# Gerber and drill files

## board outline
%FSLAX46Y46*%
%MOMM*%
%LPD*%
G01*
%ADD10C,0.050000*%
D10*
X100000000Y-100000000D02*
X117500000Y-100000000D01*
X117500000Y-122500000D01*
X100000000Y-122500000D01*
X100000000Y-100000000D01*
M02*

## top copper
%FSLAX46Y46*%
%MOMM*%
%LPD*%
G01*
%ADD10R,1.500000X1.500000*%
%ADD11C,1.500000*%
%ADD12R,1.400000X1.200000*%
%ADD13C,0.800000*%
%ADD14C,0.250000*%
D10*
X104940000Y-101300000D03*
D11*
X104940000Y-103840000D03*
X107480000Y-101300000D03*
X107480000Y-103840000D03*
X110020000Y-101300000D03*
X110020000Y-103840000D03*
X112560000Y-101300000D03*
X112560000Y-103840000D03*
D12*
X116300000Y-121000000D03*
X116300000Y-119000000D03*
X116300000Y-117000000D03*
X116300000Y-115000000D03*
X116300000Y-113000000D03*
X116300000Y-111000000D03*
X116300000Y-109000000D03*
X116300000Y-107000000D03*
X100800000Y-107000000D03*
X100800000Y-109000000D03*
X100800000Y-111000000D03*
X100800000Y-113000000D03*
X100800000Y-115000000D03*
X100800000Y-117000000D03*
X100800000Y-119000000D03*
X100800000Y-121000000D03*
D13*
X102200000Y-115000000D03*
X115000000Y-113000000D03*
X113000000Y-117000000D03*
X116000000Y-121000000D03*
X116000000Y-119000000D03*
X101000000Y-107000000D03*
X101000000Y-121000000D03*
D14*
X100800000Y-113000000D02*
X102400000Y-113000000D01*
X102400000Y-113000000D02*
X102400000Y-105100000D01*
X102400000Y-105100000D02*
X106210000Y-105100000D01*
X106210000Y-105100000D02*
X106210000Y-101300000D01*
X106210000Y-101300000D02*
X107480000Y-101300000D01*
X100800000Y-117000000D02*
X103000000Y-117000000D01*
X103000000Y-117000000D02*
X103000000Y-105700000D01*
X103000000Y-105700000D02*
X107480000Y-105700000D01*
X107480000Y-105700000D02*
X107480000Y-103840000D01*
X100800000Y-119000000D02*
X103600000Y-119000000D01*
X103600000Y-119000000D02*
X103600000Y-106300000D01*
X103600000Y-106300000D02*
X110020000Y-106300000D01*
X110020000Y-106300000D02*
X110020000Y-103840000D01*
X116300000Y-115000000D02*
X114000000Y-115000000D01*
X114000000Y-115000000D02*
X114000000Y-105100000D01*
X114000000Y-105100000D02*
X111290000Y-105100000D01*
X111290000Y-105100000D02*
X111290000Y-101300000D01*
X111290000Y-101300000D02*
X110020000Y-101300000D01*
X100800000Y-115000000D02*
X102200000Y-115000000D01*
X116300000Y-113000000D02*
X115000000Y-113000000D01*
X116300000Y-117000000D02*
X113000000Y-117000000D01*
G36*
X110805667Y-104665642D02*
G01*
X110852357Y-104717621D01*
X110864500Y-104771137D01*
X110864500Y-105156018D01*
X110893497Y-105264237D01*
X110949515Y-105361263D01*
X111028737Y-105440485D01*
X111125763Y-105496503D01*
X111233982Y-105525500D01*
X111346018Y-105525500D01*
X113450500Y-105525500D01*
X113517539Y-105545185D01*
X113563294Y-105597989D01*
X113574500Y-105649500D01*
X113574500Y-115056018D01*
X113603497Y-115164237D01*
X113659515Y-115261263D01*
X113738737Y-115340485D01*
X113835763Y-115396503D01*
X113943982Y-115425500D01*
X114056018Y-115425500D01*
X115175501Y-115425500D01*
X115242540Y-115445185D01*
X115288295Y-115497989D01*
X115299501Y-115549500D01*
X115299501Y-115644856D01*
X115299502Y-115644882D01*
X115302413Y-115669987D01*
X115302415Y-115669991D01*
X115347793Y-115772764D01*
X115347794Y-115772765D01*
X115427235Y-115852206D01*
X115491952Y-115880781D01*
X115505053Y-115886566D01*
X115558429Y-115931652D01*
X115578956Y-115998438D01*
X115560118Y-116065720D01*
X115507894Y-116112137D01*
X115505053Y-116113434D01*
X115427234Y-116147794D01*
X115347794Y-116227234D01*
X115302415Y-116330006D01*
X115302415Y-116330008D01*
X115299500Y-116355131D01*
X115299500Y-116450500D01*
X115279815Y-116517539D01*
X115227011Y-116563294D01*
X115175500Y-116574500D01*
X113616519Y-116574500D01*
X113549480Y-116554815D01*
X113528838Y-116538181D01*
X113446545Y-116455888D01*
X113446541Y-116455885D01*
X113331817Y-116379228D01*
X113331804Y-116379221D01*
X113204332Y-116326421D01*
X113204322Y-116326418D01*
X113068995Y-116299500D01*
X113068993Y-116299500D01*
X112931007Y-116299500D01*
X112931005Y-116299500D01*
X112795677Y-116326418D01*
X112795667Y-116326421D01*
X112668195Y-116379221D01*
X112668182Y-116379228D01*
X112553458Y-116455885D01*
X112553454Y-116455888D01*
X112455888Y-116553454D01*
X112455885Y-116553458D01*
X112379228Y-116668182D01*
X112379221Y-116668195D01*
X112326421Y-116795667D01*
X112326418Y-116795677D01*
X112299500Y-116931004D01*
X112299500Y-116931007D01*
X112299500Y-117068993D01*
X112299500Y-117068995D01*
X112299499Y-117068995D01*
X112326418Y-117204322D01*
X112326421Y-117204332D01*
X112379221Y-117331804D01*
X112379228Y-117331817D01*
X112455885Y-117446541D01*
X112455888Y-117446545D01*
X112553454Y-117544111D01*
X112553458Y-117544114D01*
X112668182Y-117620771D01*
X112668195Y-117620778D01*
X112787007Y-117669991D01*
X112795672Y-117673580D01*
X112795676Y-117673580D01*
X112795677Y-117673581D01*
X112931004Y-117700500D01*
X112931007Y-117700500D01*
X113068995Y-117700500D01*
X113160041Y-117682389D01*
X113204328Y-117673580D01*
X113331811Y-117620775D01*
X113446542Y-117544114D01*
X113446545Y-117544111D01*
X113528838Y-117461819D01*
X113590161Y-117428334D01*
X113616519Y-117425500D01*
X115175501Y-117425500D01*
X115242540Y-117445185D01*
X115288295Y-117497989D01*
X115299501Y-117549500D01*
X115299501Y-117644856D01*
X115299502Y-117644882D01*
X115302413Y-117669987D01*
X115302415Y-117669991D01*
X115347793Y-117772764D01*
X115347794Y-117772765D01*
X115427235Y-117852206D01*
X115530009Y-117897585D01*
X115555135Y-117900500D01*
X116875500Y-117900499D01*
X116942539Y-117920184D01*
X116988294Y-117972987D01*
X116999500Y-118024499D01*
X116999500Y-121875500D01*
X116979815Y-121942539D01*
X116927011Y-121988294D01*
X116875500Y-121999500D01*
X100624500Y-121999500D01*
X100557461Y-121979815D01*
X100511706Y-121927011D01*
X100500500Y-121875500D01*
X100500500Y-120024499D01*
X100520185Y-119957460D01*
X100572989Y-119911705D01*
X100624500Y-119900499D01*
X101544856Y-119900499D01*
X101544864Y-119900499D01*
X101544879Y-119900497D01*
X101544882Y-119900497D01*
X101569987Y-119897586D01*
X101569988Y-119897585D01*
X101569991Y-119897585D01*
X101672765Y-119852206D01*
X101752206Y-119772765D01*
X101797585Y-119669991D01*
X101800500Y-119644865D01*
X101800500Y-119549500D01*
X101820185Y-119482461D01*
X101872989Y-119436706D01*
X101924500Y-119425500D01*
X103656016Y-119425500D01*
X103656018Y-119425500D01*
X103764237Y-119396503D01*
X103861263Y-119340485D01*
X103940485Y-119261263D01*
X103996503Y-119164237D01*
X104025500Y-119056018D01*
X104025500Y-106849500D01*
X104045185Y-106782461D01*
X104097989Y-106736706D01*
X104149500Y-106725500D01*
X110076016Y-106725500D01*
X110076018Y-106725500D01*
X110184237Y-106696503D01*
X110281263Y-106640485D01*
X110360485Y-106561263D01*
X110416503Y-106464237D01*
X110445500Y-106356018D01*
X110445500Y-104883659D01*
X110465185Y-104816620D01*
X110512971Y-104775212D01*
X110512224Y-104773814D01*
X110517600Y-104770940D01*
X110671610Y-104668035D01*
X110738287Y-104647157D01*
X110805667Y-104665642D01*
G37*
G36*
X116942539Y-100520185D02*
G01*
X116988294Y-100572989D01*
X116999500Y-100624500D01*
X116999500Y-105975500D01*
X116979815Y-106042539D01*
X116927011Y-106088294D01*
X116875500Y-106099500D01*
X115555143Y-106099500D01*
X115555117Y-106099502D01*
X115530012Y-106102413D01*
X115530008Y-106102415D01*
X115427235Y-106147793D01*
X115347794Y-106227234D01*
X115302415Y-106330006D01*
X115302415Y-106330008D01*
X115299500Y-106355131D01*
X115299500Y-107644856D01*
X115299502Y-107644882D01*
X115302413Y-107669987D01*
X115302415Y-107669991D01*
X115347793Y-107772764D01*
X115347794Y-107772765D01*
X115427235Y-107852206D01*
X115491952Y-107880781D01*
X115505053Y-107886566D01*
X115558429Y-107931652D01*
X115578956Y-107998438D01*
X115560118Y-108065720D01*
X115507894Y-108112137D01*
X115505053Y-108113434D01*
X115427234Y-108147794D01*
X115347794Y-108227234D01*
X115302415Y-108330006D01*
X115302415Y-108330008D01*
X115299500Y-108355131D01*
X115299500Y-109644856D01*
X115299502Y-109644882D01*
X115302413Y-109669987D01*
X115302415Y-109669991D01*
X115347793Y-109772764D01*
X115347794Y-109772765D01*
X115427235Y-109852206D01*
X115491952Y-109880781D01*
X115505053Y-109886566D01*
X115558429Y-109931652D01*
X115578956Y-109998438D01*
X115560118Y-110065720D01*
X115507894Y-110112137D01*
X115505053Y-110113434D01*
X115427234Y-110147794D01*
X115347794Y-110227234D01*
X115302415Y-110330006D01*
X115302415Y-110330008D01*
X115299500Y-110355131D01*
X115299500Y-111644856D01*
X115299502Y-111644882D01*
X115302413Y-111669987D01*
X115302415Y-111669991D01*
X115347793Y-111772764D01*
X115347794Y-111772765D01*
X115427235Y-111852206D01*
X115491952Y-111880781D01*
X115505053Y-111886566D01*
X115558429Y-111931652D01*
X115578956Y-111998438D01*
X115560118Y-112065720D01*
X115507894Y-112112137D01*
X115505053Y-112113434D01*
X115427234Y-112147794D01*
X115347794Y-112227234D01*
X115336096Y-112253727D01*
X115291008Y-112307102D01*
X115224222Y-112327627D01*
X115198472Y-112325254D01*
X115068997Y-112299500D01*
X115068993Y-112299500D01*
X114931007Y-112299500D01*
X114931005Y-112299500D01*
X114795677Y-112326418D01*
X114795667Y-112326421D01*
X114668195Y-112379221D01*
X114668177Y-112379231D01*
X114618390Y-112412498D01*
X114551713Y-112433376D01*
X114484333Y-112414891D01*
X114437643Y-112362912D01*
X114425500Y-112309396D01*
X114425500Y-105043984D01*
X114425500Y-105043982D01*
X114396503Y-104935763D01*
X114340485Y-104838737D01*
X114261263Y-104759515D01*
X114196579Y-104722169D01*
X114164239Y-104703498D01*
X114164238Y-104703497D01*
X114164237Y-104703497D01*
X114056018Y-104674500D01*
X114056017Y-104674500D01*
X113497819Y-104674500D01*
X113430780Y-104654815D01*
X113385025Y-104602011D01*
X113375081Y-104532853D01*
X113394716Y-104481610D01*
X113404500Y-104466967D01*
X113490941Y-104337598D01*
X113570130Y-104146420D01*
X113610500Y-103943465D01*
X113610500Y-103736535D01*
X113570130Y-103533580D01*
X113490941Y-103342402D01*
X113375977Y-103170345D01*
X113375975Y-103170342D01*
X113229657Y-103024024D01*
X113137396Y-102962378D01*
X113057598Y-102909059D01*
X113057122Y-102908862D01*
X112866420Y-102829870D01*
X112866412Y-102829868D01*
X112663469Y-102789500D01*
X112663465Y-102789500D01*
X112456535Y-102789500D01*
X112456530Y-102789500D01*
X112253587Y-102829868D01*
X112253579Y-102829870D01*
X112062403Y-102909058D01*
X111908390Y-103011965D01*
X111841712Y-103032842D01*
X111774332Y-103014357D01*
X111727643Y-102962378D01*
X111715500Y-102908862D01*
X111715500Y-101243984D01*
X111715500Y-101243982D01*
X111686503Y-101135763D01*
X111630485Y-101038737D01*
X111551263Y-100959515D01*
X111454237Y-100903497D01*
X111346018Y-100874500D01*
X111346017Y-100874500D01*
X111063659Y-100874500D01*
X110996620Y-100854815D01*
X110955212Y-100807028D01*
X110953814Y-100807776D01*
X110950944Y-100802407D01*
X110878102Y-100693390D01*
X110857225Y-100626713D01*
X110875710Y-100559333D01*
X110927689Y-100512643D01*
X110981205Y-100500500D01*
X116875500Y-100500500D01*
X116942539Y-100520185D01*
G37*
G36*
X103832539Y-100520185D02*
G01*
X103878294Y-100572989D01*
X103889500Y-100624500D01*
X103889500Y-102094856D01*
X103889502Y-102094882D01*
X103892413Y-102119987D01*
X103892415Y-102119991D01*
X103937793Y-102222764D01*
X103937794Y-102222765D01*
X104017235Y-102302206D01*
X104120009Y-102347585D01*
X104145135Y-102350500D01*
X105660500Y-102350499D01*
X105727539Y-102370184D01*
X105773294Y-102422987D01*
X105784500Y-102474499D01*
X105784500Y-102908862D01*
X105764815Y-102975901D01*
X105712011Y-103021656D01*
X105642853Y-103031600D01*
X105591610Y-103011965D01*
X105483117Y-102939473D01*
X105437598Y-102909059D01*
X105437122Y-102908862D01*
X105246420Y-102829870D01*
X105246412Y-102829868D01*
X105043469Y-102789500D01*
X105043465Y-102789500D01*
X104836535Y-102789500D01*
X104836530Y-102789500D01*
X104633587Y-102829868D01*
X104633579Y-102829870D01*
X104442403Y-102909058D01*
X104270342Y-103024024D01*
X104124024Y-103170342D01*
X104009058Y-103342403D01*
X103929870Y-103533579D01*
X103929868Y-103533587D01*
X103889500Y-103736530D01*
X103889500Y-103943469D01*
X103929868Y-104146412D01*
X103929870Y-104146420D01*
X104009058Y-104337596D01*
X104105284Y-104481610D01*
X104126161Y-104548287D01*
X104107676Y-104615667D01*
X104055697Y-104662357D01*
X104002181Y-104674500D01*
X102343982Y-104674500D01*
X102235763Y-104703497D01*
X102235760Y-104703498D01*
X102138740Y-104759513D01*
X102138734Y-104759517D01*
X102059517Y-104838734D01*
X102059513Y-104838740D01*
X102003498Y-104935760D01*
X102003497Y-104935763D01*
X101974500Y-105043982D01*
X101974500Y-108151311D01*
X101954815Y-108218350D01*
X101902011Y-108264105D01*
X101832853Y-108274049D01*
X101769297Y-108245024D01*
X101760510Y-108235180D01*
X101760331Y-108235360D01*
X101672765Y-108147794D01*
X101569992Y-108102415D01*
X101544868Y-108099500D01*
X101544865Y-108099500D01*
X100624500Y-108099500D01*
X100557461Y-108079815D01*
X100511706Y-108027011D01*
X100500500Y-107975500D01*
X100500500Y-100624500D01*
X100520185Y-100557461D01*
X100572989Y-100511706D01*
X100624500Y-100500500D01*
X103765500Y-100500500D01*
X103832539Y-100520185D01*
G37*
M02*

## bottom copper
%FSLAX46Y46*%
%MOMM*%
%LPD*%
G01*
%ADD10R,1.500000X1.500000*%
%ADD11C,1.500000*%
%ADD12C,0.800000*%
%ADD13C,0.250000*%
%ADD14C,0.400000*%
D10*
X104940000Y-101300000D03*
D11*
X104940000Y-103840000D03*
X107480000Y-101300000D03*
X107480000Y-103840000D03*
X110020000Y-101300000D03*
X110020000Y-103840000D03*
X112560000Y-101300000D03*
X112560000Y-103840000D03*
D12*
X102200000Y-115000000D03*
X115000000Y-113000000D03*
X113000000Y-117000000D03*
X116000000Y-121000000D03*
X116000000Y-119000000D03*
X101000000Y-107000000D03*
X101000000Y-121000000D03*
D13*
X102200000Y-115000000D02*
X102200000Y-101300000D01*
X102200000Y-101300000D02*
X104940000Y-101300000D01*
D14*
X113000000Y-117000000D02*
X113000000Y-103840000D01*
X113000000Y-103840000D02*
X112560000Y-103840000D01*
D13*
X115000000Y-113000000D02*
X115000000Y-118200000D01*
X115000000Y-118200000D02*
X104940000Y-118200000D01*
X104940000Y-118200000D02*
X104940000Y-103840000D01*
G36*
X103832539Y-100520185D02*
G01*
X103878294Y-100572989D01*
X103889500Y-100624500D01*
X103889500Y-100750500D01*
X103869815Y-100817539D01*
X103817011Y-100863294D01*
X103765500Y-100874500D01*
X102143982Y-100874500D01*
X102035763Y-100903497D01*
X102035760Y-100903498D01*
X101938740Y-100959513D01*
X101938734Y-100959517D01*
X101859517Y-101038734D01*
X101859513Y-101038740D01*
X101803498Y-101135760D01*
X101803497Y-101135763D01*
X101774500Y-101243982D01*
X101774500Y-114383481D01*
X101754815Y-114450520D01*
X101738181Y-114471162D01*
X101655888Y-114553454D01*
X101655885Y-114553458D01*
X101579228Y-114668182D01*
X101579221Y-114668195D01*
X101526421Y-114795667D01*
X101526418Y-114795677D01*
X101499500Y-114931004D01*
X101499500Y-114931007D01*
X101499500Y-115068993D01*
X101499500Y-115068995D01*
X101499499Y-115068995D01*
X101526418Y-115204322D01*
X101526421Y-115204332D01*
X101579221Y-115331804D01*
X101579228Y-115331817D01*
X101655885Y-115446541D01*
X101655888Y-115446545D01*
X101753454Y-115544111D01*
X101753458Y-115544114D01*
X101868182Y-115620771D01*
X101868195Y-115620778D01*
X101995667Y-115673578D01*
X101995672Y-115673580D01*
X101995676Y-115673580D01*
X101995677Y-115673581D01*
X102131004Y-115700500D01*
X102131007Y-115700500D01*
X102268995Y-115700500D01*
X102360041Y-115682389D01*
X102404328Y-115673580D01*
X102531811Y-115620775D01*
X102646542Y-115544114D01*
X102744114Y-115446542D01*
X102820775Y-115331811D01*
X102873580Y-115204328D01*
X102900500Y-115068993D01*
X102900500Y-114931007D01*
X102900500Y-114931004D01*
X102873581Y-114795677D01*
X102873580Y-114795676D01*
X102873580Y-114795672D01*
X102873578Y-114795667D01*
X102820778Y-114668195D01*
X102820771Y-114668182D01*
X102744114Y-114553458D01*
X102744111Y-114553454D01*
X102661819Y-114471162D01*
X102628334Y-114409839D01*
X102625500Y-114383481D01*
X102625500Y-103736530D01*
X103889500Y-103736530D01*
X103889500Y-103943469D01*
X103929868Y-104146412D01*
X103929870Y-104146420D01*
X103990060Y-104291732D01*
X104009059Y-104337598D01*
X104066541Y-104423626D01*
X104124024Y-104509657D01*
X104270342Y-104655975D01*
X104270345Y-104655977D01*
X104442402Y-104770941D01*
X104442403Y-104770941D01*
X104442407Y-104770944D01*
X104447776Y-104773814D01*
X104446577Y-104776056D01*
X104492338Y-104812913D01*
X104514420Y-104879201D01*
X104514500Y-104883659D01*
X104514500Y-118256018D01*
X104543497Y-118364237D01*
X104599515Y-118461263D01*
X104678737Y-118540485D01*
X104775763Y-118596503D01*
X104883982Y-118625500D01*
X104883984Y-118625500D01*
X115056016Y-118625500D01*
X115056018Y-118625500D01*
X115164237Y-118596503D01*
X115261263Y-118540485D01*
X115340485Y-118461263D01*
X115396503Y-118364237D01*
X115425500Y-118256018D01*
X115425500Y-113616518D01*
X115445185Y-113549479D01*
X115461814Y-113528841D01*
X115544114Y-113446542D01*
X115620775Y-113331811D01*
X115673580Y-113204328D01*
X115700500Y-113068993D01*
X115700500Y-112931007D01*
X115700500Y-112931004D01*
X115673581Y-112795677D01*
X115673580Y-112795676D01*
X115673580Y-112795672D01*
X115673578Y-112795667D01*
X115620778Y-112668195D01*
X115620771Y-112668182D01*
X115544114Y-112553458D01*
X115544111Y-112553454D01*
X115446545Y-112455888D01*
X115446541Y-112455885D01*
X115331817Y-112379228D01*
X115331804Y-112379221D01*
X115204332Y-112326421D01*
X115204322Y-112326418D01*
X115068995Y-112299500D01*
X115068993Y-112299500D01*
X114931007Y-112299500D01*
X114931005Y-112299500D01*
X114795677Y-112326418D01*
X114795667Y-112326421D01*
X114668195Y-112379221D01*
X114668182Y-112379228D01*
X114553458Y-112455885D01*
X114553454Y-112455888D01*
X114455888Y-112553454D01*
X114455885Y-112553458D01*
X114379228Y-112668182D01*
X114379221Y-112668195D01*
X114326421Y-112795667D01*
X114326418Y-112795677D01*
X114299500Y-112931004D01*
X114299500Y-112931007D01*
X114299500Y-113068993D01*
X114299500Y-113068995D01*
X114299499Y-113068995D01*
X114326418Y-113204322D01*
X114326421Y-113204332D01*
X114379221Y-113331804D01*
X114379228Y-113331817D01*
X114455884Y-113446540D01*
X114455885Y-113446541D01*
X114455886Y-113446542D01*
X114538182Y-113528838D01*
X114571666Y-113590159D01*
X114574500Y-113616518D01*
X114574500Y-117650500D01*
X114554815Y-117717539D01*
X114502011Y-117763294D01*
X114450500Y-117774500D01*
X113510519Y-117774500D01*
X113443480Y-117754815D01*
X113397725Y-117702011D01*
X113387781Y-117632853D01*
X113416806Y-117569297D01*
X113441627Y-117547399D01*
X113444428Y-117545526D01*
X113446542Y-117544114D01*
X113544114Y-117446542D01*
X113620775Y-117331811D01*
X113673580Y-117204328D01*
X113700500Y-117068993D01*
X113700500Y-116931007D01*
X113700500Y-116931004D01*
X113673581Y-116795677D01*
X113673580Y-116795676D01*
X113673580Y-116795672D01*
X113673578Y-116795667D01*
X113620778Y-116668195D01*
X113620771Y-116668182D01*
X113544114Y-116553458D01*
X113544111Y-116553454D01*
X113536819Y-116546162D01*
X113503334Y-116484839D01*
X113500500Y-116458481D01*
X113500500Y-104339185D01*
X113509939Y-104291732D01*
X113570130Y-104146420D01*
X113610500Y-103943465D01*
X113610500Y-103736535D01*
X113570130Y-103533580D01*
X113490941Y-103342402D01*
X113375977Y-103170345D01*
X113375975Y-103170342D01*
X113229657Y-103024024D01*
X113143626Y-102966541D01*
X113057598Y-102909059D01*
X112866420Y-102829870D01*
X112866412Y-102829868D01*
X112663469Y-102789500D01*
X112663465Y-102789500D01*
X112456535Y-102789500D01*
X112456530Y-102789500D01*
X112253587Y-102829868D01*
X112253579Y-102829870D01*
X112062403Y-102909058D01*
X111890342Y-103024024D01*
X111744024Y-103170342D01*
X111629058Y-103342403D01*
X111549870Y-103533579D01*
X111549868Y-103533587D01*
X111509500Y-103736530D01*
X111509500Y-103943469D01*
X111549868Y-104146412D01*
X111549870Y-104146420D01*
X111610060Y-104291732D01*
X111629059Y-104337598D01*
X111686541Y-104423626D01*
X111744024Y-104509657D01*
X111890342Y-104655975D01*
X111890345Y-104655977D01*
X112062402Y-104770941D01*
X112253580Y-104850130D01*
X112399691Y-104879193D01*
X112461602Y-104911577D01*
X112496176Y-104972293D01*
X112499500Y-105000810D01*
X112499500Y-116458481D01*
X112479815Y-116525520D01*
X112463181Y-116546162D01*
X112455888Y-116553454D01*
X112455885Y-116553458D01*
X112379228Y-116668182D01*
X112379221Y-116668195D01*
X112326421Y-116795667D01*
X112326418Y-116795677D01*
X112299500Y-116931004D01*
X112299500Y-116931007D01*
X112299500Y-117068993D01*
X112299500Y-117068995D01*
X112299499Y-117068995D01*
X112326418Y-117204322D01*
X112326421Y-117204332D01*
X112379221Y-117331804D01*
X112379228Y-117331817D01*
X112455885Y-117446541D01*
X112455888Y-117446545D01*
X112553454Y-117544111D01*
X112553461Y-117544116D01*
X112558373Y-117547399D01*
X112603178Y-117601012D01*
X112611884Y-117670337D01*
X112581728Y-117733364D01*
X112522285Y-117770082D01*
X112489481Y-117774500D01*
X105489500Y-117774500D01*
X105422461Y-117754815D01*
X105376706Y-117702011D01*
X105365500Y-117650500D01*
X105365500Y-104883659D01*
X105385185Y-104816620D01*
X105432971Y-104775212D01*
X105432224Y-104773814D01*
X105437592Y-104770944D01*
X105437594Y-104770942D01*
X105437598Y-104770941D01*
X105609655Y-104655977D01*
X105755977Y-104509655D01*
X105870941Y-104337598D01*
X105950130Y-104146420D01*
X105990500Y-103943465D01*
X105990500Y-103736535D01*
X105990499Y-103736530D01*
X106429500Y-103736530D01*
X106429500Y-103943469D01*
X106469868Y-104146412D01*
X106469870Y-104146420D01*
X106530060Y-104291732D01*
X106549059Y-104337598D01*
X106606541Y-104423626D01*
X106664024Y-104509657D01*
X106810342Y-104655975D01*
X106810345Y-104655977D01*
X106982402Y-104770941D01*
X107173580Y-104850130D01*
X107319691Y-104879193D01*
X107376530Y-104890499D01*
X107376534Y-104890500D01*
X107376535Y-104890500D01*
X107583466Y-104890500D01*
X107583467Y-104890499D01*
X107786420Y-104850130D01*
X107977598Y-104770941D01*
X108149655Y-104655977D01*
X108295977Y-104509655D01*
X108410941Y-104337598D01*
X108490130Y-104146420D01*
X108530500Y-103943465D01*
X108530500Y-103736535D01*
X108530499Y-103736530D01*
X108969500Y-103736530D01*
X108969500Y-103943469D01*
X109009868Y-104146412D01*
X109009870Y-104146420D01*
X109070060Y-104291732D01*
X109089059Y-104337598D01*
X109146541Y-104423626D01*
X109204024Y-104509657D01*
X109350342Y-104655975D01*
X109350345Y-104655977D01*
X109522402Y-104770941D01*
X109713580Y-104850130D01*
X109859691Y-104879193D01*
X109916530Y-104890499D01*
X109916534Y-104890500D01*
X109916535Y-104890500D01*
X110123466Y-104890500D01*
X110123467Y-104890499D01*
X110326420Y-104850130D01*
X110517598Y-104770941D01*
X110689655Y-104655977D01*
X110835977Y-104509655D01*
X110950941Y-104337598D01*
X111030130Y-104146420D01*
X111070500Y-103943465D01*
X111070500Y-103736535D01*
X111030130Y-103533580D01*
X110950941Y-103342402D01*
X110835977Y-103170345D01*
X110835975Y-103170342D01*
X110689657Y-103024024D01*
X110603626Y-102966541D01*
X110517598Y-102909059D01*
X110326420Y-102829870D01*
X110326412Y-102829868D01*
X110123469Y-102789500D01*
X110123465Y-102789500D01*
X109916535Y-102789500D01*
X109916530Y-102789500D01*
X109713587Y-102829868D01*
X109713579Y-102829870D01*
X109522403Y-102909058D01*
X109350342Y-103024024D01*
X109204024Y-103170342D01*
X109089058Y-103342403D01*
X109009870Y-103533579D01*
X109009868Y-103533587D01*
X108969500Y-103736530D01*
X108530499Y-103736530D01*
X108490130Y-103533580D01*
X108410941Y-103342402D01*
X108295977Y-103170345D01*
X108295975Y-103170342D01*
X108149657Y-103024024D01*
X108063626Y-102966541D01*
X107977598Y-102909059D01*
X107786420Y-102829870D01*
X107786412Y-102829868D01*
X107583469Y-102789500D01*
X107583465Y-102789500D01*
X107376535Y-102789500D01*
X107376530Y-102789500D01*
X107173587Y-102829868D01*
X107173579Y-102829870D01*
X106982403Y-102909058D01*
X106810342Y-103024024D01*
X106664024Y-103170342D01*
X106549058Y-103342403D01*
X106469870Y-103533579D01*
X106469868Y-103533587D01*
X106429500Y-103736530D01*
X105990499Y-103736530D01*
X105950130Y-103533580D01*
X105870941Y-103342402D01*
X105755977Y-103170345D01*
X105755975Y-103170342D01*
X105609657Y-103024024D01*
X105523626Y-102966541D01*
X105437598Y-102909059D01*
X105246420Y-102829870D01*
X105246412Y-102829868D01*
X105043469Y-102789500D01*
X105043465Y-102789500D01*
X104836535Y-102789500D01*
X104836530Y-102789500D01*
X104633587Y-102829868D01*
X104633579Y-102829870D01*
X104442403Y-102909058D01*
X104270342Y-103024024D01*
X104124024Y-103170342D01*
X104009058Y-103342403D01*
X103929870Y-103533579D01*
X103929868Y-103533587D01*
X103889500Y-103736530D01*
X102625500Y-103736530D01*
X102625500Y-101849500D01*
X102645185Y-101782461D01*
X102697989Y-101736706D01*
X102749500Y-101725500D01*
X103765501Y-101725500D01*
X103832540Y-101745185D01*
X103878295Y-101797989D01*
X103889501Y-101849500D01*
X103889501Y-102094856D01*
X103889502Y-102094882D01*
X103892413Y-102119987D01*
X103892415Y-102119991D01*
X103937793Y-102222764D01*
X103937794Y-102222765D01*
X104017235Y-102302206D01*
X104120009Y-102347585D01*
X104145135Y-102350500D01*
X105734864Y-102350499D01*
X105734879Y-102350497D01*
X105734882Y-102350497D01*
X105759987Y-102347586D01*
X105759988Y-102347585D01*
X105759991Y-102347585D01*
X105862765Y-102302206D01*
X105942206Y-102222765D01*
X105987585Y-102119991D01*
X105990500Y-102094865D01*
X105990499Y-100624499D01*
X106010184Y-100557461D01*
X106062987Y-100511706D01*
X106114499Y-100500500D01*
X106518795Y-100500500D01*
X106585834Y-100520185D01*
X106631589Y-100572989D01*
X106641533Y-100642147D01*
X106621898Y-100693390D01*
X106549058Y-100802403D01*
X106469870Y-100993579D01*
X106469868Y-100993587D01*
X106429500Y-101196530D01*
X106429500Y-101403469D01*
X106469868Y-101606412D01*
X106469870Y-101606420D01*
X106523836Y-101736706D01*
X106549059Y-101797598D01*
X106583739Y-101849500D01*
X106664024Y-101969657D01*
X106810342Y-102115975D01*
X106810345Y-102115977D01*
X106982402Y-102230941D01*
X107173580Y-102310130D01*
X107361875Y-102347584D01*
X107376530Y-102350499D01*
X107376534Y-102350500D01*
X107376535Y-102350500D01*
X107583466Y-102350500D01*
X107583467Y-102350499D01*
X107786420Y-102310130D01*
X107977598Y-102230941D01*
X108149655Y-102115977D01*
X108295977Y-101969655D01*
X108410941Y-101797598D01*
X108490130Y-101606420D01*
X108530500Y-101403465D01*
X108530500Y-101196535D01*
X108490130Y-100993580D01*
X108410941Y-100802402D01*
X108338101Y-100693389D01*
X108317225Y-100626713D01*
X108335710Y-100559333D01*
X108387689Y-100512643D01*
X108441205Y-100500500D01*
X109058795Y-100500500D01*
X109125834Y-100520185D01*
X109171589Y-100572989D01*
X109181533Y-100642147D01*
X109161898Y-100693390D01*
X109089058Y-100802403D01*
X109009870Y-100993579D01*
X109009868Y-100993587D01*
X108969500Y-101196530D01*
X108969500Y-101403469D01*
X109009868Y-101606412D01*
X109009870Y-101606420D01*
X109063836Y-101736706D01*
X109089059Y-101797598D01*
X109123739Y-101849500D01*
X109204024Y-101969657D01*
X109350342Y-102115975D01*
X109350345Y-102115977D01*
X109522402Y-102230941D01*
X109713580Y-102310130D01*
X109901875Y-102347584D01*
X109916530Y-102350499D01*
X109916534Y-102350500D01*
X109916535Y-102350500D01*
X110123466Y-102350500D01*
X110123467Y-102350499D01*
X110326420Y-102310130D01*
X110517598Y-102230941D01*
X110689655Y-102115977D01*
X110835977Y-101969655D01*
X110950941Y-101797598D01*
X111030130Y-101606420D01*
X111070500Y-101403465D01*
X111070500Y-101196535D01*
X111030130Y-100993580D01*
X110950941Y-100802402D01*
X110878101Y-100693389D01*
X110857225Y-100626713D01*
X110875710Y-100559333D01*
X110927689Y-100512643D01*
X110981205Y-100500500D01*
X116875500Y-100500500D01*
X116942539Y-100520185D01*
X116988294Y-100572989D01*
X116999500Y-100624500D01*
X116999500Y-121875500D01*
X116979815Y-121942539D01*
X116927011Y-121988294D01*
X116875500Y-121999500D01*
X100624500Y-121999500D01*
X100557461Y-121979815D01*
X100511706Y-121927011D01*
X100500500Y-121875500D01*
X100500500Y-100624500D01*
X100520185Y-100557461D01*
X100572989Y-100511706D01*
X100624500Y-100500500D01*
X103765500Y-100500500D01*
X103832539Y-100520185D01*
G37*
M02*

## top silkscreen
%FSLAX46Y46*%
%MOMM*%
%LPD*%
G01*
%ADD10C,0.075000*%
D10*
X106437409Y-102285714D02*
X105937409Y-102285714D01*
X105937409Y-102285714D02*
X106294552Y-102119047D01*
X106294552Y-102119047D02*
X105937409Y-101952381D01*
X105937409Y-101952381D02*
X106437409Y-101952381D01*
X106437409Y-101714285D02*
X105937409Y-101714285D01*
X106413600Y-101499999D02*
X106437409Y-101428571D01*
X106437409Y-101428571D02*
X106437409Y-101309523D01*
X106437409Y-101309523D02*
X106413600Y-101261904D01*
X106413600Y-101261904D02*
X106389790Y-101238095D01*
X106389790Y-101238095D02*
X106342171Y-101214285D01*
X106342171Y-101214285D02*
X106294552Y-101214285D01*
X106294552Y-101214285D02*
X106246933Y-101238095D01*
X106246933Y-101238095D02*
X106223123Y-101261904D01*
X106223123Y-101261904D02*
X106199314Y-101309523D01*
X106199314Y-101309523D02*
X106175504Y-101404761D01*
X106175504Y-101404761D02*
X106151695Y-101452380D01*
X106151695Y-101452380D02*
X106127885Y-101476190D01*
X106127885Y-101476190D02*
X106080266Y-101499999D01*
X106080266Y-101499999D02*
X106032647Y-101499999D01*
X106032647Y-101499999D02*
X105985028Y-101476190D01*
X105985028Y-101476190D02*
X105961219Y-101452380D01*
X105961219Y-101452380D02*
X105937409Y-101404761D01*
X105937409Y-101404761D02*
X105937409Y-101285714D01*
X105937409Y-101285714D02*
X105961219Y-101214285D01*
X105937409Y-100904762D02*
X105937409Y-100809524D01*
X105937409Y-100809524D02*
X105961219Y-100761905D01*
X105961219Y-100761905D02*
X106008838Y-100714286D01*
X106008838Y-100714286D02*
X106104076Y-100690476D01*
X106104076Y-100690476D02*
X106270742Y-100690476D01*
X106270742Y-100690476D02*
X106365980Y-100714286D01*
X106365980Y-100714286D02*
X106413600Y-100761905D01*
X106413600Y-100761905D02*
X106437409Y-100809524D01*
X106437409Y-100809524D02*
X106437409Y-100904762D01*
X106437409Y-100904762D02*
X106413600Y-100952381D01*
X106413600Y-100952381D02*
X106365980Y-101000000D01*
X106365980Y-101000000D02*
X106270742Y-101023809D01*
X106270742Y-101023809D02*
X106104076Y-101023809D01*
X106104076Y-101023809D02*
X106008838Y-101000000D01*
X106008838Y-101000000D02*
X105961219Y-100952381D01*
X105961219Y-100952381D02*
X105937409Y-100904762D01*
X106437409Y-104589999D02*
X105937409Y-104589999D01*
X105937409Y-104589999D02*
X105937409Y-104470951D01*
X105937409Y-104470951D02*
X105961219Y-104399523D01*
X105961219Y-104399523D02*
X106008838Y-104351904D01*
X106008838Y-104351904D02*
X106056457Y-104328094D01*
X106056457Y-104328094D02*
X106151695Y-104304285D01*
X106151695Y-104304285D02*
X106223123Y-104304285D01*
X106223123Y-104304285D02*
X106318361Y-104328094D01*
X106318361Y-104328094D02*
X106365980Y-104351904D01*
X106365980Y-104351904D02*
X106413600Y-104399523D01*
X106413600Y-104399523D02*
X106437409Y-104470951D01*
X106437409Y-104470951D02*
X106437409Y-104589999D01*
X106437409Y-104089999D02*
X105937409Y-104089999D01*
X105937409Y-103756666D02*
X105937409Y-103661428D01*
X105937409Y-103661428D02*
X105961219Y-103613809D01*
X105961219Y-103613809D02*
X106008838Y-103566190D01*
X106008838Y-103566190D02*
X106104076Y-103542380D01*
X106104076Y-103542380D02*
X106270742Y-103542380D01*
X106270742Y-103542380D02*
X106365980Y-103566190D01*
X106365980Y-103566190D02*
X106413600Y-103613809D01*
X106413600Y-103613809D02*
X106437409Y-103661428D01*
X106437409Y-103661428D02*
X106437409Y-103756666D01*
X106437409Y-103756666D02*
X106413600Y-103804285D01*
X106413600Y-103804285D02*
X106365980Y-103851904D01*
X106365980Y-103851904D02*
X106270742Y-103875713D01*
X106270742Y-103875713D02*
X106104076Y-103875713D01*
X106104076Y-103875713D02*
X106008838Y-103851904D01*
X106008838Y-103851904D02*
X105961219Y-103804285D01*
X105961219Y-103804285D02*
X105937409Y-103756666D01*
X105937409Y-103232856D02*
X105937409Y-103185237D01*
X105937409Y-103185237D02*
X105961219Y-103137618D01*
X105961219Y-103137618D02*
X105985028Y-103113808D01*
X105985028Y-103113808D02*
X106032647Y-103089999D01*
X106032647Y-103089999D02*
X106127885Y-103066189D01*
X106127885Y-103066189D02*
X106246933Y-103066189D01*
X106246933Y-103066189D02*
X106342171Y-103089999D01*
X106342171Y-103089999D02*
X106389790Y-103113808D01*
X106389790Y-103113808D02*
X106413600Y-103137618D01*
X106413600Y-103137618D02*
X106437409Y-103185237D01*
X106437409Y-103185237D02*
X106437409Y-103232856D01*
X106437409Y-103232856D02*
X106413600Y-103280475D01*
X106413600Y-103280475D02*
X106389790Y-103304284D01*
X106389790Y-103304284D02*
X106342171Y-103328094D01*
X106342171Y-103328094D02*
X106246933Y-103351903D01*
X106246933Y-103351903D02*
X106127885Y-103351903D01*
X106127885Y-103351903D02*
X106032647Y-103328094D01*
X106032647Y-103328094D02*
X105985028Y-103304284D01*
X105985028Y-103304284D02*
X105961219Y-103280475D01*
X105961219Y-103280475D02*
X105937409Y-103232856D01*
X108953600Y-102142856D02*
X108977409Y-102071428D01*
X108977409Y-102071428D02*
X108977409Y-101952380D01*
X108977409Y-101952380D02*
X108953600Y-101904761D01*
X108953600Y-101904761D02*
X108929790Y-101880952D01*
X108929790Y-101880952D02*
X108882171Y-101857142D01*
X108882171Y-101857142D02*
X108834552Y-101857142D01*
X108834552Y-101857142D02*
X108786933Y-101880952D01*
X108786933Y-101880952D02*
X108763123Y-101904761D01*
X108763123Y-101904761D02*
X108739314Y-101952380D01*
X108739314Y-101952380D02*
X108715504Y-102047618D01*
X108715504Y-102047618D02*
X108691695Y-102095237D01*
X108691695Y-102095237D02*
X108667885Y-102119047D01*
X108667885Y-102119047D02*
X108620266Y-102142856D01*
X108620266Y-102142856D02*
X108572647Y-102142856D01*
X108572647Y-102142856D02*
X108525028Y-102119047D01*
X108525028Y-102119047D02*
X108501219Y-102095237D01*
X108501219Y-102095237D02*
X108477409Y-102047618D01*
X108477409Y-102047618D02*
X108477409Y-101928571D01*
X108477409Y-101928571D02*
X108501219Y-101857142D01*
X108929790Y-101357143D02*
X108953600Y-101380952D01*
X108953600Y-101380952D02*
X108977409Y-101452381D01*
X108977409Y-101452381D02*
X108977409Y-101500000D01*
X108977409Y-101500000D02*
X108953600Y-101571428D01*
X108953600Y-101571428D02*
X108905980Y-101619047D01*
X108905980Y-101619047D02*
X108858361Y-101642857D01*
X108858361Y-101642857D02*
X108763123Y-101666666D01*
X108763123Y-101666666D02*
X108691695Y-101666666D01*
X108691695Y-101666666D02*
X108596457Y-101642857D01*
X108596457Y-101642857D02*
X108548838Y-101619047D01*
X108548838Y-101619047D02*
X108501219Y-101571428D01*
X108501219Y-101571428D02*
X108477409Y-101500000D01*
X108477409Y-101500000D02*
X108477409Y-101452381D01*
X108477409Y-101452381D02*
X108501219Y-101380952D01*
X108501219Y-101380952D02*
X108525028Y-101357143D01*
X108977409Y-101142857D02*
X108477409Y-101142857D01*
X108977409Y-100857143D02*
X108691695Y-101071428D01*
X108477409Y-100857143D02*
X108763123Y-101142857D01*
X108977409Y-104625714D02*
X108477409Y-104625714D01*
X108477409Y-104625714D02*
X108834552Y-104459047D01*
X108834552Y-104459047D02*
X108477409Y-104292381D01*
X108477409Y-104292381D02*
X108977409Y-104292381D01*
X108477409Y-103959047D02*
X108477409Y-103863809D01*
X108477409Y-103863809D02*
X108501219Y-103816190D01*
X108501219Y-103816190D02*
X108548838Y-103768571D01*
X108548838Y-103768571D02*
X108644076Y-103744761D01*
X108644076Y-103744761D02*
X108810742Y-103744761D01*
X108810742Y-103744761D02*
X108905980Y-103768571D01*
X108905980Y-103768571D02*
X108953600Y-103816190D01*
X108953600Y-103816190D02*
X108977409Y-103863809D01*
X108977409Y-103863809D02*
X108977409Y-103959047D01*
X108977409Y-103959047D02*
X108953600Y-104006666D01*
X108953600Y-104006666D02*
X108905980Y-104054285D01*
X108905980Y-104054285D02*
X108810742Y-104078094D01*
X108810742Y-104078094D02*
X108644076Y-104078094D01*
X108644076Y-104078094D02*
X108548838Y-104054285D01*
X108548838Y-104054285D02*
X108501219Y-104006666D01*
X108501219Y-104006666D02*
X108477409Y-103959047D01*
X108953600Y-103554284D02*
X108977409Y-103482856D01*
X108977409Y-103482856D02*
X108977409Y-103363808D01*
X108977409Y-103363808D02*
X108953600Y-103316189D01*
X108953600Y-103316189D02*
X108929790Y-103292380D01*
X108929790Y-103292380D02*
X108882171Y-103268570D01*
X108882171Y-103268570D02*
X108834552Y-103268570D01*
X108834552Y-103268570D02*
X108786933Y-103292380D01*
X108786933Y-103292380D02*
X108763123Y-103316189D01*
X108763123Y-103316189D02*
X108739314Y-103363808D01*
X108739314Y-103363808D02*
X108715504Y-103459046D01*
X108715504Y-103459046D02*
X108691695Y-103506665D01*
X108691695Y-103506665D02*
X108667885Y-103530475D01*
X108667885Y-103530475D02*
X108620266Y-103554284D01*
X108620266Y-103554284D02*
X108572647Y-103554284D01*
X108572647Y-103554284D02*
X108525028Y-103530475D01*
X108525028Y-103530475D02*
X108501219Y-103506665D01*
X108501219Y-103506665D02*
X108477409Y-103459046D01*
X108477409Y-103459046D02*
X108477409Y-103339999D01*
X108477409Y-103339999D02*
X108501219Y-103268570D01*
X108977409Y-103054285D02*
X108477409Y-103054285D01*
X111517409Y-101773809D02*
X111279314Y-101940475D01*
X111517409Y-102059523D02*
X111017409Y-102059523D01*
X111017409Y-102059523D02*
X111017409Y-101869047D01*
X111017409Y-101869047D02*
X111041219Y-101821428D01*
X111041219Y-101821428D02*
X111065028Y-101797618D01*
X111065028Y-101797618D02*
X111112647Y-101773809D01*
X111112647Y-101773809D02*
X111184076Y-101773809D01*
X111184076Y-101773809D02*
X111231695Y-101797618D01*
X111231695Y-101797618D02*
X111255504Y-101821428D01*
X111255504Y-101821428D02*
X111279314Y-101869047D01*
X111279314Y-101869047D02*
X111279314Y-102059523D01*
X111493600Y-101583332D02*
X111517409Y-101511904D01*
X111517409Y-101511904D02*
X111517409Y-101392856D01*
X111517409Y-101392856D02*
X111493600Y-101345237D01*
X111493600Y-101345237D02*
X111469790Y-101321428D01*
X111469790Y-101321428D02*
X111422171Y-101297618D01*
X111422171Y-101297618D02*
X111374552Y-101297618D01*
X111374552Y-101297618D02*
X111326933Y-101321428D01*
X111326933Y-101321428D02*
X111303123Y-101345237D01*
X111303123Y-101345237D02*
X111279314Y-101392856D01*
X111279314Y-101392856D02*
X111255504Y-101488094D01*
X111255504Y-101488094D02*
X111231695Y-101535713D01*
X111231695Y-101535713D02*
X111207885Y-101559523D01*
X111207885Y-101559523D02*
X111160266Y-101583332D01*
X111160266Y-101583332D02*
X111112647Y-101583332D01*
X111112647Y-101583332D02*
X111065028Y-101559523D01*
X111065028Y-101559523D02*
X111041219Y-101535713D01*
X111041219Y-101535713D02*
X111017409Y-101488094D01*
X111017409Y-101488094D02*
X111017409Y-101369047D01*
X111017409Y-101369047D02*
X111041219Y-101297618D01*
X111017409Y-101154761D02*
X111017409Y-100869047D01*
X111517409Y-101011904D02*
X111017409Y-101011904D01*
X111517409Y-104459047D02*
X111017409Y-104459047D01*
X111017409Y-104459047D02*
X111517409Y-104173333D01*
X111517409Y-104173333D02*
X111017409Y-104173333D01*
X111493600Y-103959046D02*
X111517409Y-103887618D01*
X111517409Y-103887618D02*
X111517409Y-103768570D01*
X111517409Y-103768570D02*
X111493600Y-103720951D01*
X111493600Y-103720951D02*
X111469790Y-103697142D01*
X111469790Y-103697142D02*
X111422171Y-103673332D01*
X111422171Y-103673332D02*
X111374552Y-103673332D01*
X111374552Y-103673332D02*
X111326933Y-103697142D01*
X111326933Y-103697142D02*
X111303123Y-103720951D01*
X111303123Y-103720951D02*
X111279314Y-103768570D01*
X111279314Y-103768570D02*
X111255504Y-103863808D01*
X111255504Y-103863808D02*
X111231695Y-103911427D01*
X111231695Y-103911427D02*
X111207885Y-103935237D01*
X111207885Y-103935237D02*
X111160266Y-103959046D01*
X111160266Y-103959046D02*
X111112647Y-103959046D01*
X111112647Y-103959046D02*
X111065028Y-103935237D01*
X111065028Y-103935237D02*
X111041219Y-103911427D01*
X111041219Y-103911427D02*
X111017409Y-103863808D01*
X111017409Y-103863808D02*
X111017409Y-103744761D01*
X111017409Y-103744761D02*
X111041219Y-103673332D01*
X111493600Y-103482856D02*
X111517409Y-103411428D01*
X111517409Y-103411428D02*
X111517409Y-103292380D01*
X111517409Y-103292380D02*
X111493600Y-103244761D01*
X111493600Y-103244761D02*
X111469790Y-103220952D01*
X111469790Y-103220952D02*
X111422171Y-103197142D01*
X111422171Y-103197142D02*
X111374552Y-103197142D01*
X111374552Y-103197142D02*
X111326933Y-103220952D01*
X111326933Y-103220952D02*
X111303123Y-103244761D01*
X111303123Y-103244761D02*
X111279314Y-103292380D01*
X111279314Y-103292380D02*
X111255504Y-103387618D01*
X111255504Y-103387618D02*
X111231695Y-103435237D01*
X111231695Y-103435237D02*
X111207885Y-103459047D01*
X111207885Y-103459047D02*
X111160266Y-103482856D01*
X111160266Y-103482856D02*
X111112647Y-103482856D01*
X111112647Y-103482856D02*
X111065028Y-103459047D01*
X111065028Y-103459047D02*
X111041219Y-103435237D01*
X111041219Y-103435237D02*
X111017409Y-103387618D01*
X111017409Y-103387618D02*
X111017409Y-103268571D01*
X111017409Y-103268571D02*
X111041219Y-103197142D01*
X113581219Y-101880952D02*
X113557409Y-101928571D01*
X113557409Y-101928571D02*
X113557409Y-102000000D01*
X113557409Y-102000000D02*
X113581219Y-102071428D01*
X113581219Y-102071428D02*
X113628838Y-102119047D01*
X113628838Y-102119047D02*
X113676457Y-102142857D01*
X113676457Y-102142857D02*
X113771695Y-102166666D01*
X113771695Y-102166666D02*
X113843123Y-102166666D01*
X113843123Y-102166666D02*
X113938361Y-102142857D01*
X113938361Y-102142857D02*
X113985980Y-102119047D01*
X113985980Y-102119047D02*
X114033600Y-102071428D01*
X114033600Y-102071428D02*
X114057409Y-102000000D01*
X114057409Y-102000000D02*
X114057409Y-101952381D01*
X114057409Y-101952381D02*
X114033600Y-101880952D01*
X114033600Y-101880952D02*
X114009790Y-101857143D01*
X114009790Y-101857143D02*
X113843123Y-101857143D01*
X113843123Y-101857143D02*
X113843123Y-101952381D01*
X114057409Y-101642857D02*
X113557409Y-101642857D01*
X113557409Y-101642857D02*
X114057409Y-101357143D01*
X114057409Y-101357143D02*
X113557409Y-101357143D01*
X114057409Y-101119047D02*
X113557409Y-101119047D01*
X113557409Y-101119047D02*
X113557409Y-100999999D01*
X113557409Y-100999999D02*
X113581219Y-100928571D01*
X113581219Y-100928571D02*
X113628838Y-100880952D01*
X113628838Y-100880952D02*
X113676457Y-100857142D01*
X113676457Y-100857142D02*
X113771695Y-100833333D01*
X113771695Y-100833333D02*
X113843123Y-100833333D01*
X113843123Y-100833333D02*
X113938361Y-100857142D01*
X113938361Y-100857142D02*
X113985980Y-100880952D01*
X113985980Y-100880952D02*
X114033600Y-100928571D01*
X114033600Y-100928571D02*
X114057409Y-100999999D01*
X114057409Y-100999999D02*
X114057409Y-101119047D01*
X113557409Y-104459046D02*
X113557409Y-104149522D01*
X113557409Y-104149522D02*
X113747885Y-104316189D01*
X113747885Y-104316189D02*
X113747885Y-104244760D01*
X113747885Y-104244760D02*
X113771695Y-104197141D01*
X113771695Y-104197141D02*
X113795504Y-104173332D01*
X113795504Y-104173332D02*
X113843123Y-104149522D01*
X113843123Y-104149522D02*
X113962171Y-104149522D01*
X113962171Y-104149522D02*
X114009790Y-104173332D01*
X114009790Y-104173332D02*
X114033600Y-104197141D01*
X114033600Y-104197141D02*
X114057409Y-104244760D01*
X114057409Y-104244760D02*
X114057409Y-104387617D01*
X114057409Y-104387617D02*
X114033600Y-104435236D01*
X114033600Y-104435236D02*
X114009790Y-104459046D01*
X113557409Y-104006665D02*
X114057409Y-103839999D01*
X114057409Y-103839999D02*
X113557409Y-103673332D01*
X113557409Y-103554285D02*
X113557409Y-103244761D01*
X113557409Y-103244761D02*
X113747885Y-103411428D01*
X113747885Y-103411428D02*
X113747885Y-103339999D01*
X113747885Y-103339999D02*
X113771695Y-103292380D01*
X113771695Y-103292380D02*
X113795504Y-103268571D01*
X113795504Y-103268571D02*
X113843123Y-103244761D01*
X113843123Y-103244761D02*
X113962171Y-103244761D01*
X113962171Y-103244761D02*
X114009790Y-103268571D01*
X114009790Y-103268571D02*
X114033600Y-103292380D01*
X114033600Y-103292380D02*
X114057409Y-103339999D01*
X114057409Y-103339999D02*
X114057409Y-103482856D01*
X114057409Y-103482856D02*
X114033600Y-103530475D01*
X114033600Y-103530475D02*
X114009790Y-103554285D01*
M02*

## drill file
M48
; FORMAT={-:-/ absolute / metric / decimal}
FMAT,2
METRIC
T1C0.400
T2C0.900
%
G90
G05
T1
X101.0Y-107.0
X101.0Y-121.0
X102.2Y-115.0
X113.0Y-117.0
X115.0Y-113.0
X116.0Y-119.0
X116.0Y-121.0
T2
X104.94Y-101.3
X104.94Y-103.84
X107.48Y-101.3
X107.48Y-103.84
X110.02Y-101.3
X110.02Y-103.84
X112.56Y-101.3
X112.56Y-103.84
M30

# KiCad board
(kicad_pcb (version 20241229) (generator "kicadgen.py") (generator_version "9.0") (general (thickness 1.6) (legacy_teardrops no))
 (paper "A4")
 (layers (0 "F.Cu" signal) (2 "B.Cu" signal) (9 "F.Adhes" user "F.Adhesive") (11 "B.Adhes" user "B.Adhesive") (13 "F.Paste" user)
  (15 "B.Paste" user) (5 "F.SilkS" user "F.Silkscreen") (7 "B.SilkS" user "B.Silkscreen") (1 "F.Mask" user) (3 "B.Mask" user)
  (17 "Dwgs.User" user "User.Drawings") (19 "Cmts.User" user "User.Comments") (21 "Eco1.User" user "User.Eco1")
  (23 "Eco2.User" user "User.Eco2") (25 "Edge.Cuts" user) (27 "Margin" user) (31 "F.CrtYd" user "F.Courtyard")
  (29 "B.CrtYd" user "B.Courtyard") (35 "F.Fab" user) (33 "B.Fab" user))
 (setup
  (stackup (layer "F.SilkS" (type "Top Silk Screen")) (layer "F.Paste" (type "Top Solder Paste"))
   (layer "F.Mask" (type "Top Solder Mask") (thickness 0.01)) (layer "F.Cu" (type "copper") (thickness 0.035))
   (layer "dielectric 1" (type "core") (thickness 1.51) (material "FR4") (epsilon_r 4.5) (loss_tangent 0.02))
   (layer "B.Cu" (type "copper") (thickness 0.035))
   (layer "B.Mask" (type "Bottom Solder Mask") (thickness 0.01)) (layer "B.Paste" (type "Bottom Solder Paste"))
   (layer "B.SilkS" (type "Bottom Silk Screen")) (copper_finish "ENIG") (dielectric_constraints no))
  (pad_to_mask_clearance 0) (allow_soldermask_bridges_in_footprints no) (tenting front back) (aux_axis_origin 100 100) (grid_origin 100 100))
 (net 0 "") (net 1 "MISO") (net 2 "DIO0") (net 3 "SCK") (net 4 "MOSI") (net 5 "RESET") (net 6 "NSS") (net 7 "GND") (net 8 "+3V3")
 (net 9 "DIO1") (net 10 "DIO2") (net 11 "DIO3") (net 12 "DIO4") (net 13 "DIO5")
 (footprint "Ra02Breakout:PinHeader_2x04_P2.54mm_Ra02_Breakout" (layer "F.Cu") (at 104.94 101.3)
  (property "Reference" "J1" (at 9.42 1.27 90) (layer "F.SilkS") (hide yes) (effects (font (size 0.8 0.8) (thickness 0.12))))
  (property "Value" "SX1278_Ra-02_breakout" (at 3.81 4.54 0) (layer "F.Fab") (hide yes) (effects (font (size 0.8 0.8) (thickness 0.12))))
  (pad "1" thru_hole rect (at 0 0) (size 1.5 1.5) (drill 0.9) (layers "*.Cu" "*.Mask") (remove_unused_layers no) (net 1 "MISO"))
  (pad "2" thru_hole circle (at 0 2.54) (size 1.5 1.5) (drill 0.9) (layers "*.Cu" "*.Mask") (remove_unused_layers no) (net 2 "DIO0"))
  (pad "3" thru_hole circle (at 2.54 0) (size 1.5 1.5) (drill 0.9) (layers "*.Cu" "*.Mask") (remove_unused_layers no) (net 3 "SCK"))
  (pad "4" thru_hole circle (at 2.54 2.54) (size 1.5 1.5) (drill 0.9) (layers "*.Cu" "*.Mask") (remove_unused_layers no) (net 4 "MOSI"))
  (pad "5" thru_hole circle (at 5.08 0) (size 1.5 1.5) (drill 0.9) (layers "*.Cu" "*.Mask") (remove_unused_layers no) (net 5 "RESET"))
  (pad "6" thru_hole circle (at 5.08 2.54) (size 1.5 1.5) (drill 0.9) (layers "*.Cu" "*.Mask") (remove_unused_layers no) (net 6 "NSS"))
  (pad "7" thru_hole circle (at 7.62 0) (size 1.5 1.5) (drill 0.9) (layers "*.Cu" "*.Mask") (remove_unused_layers no) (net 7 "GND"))
  (pad "8" thru_hole circle (at 7.62 2.54) (size 1.5 1.5) (drill 0.9) (layers "*.Cu" "*.Mask") (remove_unused_layers no) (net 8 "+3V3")))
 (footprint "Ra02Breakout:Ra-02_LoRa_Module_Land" (layer "F.Cu") (at 100.2 105.5)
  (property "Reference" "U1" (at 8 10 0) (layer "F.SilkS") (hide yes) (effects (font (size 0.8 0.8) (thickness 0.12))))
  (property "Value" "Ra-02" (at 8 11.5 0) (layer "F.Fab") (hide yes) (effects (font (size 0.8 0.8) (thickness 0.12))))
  (pad "1" smd rect (at 16.1 15.5) (size 1.4 1.2) (layers "F.Cu" "F.Mask" "F.Paste") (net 7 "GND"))
  (pad "2" smd rect (at 16.1 13.5) (size 1.4 1.2) (layers "F.Cu" "F.Mask" "F.Paste") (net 7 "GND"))
  (pad "3" smd rect (at 16.1 11.5) (size 1.4 1.2) (layers "F.Cu" "F.Mask" "F.Paste") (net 8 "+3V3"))
  (pad "4" smd rect (at 16.1 9.5) (size 1.4 1.2) (layers "F.Cu" "F.Mask" "F.Paste") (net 5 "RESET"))
  (pad "5" smd rect (at 16.1 7.5) (size 1.4 1.2) (layers "F.Cu" "F.Mask" "F.Paste") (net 2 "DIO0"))
  (pad "6" smd rect (at 16.1 5.5) (size 1.4 1.2) (layers "F.Cu" "F.Mask" "F.Paste") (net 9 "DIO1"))
  (pad "7" smd rect (at 16.1 3.5) (size 1.4 1.2) (layers "F.Cu" "F.Mask" "F.Paste") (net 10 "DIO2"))
  (pad "8" smd rect (at 16.1 1.5) (size 1.4 1.2) (layers "F.Cu" "F.Mask" "F.Paste") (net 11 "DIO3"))
  (pad "9" smd rect (at 0.6 1.5) (size 1.4 1.2) (layers "F.Cu" "F.Mask" "F.Paste") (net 7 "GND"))
  (pad "10" smd rect (at 0.6 3.5) (size 1.4 1.2) (layers "F.Cu" "F.Mask" "F.Paste") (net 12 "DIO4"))
  (pad "11" smd rect (at 0.6 5.5) (size 1.4 1.2) (layers "F.Cu" "F.Mask" "F.Paste") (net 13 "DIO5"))
  (pad "12" smd rect (at 0.6 7.5) (size 1.4 1.2) (layers "F.Cu" "F.Mask" "F.Paste") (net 3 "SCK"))
  (pad "13" smd rect (at 0.6 9.5) (size 1.4 1.2) (layers "F.Cu" "F.Mask" "F.Paste") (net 1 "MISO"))
  (pad "14" smd rect (at 0.6 11.5) (size 1.4 1.2) (layers "F.Cu" "F.Mask" "F.Paste") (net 4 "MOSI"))
  (pad "15" smd rect (at 0.6 13.5) (size 1.4 1.2) (layers "F.Cu" "F.Mask" "F.Paste") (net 6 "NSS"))
  (pad "16" smd rect (at 0.6 15.5) (size 1.4 1.2) (layers "F.Cu" "F.Mask" "F.Paste") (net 7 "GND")))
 (gr_rect (start 100 100) (end 117.5 122.5) (stroke (width 0.05) (type solid)) (fill no) (layer "Edge.Cuts"))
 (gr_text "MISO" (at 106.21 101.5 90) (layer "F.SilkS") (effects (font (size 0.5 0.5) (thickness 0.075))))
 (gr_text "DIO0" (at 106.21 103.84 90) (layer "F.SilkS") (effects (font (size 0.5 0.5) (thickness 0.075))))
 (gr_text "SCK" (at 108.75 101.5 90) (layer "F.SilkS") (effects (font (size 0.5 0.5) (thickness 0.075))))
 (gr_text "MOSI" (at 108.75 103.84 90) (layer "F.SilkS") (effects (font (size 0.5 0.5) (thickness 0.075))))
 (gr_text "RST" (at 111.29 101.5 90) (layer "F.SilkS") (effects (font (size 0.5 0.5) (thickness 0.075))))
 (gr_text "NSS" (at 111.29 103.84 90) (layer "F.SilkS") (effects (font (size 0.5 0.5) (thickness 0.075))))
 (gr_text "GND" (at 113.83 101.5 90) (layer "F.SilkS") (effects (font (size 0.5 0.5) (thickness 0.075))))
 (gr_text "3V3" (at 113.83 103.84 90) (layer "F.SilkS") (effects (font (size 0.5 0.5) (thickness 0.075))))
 (segment (start 100.8 113) (end 102.4 113) (width 0.25) (layer "F.Cu") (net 3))
 (segment (start 102.4 113) (end 102.4 105.1) (width 0.25) (layer "F.Cu") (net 3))
 (segment (start 102.4 105.1) (end 106.21 105.1) (width 0.25) (layer "F.Cu") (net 3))
 (segment (start 106.21 105.1) (end 106.21 101.3) (width 0.25) (layer "F.Cu") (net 3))
 (segment (start 106.21 101.3) (end 107.48 101.3) (width 0.25) (layer "F.Cu") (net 3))
 (segment (start 100.8 117) (end 103 117) (width 0.25) (layer "F.Cu") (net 4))
 (segment (start 103 117) (end 103 105.7) (width 0.25) (layer "F.Cu") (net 4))
 (segment (start 103 105.7) (end 107.48 105.7) (width 0.25) (layer "F.Cu") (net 4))
 (segment (start 107.48 105.7) (end 107.48 103.84) (width 0.25) (layer "F.Cu") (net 4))
 (segment (start 100.8 119) (end 103.6 119) (width 0.25) (layer "F.Cu") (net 6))
 (segment (start 103.6 119) (end 103.6 106.3) (width 0.25) (layer "F.Cu") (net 6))
 (segment (start 103.6 106.3) (end 110.02 106.3) (width 0.25) (layer "F.Cu") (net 6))
 (segment (start 110.02 106.3) (end 110.02 103.84) (width 0.25) (layer "F.Cu") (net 6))
 (segment (start 116.3 115) (end 114 115) (width 0.25) (layer "F.Cu") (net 5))
 (segment (start 114 115) (end 114 105.1) (width 0.25) (layer "F.Cu") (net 5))
 (segment (start 114 105.1) (end 111.29 105.1) (width 0.25) (layer "F.Cu") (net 5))
 (segment (start 111.29 105.1) (end 111.29 101.3) (width 0.25) (layer "F.Cu") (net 5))
 (segment (start 111.29 101.3) (end 110.02 101.3) (width 0.25) (layer "F.Cu") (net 5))
 (segment (start 100.8 115) (end 102.2 115) (width 0.25) (layer "F.Cu") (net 1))
 (segment (start 116.3 113) (end 115 113) (width 0.25) (layer "F.Cu") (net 2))
 (segment (start 116.3 117) (end 113 117) (width 0.25) (layer "F.Cu") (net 8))
 (segment (start 102.2 115) (end 102.2 101.3) (width 0.25) (layer "B.Cu") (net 1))
 (segment (start 102.2 101.3) (end 104.94 101.3) (width 0.25) (layer "B.Cu") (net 1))
 (segment (start 113 117) (end 113 103.84) (width 0.4) (layer "B.Cu") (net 8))
 (segment (start 113 103.84) (end 112.56 103.84) (width 0.4) (layer "B.Cu") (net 8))
 (segment (start 115 113) (end 115 118.2) (width 0.25) (layer "B.Cu") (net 2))
 (segment (start 115 118.2) (end 104.94 118.2) (width 0.25) (layer "B.Cu") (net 2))
 (segment (start 104.94 118.2) (end 104.94 103.84) (width 0.25) (layer "B.Cu") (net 2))
 (via (at 102.2 115) (size 0.8) (drill 0.4) (layers "F.Cu" "B.Cu") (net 1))
 (via (at 115 113) (size 0.8) (drill 0.4) (layers "F.Cu" "B.Cu") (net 2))
 (via (at 113 117) (size 0.8) (drill 0.4) (layers "F.Cu" "B.Cu") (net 8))
 (via (at 116 121) (size 0.8) (drill 0.4) (layers "F.Cu" "B.Cu") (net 7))
 (via (at 116 119) (size 0.8) (drill 0.4) (layers "F.Cu" "B.Cu") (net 7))
 (via (at 101 107) (size 0.8) (drill 0.4) (layers "F.Cu" "B.Cu") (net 7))
 (via (at 101 121) (size 0.8) (drill 0.4) (layers "F.Cu" "B.Cu") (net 7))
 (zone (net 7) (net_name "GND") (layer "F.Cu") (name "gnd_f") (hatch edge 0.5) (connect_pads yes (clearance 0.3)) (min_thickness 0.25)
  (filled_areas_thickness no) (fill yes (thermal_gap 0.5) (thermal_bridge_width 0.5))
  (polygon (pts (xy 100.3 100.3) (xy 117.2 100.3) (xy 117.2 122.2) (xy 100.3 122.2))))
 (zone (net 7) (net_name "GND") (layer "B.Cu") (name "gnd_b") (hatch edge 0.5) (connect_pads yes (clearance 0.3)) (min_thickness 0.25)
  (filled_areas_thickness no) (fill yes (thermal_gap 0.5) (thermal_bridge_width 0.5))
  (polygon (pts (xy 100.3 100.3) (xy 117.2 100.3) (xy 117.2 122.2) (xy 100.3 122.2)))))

